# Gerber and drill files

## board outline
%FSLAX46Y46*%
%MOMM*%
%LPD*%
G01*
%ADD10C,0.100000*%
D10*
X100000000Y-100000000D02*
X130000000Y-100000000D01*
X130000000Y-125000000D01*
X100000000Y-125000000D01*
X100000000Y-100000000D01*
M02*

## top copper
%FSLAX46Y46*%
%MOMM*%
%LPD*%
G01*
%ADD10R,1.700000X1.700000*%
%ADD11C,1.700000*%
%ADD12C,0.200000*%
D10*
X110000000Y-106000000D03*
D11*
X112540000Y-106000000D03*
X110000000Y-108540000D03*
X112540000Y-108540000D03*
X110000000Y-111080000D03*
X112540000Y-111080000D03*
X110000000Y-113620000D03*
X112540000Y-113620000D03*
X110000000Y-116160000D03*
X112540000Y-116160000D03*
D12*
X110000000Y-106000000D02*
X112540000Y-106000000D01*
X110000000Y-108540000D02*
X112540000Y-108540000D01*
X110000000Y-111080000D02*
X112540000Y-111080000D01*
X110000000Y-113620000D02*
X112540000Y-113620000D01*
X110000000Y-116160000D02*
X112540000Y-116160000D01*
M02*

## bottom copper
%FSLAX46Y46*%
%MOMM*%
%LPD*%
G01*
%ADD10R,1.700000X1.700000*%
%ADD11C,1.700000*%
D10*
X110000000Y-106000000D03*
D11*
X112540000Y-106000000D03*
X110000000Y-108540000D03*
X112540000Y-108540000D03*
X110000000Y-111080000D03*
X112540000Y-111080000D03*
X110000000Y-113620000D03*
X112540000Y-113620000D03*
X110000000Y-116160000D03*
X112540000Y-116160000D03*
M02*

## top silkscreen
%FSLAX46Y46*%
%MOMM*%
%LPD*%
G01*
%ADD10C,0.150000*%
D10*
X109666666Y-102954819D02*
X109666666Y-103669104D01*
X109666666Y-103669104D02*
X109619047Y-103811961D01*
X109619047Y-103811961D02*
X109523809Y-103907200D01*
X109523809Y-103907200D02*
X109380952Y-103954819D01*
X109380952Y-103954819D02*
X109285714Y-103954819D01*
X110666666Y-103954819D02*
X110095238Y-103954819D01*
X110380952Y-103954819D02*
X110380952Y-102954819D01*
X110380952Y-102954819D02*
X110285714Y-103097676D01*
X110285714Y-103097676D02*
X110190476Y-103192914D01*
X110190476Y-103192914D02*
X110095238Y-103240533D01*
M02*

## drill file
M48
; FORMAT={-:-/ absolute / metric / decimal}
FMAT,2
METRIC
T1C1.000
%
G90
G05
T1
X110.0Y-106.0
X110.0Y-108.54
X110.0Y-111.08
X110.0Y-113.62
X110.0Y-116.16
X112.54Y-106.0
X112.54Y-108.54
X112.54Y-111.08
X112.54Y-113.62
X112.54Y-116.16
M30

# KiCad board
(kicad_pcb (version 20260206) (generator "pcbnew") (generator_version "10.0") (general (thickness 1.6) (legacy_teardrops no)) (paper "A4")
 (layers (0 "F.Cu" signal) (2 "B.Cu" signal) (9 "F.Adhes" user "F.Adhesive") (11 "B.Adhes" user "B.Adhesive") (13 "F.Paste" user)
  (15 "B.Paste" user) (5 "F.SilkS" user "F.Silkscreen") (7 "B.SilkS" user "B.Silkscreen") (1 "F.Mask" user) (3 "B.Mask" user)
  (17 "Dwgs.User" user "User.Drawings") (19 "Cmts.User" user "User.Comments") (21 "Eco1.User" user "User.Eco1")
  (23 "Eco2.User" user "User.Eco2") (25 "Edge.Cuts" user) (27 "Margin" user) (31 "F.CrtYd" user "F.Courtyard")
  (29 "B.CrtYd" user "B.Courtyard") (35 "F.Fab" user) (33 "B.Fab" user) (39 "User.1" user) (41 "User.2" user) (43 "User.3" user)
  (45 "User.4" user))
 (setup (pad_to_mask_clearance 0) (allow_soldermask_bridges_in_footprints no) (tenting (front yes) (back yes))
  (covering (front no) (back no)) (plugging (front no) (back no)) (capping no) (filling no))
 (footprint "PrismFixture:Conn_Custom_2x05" (layer "F.Cu") (at 110 106)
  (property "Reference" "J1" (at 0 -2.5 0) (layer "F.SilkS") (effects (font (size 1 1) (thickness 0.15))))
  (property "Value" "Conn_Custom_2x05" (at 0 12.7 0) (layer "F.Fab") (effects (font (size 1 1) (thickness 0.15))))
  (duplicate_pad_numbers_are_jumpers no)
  (pad "1" thru_hole rect (at 0 0) (size 1.7 1.7) (drill 1) (layers "*.Cu" "*.Mask") (remove_unused_layers no) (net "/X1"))
  (pad "2" thru_hole circle (at 2.54 0) (size 1.7 1.7) (drill 1) (layers "*.Cu" "*.Mask") (remove_unused_layers no) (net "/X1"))
  (pad "3" thru_hole circle (at 0 2.54) (size 1.7 1.7) (drill 1) (layers "*.Cu" "*.Mask") (remove_unused_layers no) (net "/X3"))
  (pad "4" thru_hole circle (at 2.54 2.54) (size 1.7 1.7) (drill 1) (layers "*.Cu" "*.Mask") (remove_unused_layers no) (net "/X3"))
  (pad "5" thru_hole circle (at 0 5.08) (size 1.7 1.7) (drill 1) (layers "*.Cu" "*.Mask") (remove_unused_layers no) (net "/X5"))
  (pad "6" thru_hole circle (at 2.54 5.08) (size 1.7 1.7) (drill 1) (layers "*.Cu" "*.Mask") (remove_unused_layers no) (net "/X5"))
  (pad "7" thru_hole circle (at 0 7.62) (size 1.7 1.7) (drill 1) (layers "*.Cu" "*.Mask") (remove_unused_layers no) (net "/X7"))
  (pad "8" thru_hole circle (at 2.54 7.62) (size 1.7 1.7) (drill 1) (layers "*.Cu" "*.Mask") (remove_unused_layers no) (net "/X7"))
  (pad "9" thru_hole circle (at 0 10.16) (size 1.7 1.7) (drill 1) (layers "*.Cu" "*.Mask") (remove_unused_layers no) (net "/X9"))
  (pad "10" thru_hole circle (at 2.54 10.16) (size 1.7 1.7) (drill 1) (layers "*.Cu" "*.Mask") (remove_unused_layers no) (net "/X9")))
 (gr_rect (start 100 100) (end 130 125) (stroke (width 0.1) (type solid)) (fill no) (layer "Edge.Cuts"))
 (segment (start 110 106) (end 112.54 106) (width 0.2) (layer "F.Cu") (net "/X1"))
 (segment (start 110 108.54) (end 112.54 108.54) (width 0.2) (layer "F.Cu") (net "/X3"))
 (segment (start 110 111.08) (end 112.54 111.08) (width 0.2) (layer "F.Cu") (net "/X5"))
 (segment (start 110 113.62) (end 112.54 113.62) (width 0.2) (layer "F.Cu") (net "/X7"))
 (segment (start 110 116.16) (end 112.54 116.16) (width 0.2) (layer "F.Cu") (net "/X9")))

